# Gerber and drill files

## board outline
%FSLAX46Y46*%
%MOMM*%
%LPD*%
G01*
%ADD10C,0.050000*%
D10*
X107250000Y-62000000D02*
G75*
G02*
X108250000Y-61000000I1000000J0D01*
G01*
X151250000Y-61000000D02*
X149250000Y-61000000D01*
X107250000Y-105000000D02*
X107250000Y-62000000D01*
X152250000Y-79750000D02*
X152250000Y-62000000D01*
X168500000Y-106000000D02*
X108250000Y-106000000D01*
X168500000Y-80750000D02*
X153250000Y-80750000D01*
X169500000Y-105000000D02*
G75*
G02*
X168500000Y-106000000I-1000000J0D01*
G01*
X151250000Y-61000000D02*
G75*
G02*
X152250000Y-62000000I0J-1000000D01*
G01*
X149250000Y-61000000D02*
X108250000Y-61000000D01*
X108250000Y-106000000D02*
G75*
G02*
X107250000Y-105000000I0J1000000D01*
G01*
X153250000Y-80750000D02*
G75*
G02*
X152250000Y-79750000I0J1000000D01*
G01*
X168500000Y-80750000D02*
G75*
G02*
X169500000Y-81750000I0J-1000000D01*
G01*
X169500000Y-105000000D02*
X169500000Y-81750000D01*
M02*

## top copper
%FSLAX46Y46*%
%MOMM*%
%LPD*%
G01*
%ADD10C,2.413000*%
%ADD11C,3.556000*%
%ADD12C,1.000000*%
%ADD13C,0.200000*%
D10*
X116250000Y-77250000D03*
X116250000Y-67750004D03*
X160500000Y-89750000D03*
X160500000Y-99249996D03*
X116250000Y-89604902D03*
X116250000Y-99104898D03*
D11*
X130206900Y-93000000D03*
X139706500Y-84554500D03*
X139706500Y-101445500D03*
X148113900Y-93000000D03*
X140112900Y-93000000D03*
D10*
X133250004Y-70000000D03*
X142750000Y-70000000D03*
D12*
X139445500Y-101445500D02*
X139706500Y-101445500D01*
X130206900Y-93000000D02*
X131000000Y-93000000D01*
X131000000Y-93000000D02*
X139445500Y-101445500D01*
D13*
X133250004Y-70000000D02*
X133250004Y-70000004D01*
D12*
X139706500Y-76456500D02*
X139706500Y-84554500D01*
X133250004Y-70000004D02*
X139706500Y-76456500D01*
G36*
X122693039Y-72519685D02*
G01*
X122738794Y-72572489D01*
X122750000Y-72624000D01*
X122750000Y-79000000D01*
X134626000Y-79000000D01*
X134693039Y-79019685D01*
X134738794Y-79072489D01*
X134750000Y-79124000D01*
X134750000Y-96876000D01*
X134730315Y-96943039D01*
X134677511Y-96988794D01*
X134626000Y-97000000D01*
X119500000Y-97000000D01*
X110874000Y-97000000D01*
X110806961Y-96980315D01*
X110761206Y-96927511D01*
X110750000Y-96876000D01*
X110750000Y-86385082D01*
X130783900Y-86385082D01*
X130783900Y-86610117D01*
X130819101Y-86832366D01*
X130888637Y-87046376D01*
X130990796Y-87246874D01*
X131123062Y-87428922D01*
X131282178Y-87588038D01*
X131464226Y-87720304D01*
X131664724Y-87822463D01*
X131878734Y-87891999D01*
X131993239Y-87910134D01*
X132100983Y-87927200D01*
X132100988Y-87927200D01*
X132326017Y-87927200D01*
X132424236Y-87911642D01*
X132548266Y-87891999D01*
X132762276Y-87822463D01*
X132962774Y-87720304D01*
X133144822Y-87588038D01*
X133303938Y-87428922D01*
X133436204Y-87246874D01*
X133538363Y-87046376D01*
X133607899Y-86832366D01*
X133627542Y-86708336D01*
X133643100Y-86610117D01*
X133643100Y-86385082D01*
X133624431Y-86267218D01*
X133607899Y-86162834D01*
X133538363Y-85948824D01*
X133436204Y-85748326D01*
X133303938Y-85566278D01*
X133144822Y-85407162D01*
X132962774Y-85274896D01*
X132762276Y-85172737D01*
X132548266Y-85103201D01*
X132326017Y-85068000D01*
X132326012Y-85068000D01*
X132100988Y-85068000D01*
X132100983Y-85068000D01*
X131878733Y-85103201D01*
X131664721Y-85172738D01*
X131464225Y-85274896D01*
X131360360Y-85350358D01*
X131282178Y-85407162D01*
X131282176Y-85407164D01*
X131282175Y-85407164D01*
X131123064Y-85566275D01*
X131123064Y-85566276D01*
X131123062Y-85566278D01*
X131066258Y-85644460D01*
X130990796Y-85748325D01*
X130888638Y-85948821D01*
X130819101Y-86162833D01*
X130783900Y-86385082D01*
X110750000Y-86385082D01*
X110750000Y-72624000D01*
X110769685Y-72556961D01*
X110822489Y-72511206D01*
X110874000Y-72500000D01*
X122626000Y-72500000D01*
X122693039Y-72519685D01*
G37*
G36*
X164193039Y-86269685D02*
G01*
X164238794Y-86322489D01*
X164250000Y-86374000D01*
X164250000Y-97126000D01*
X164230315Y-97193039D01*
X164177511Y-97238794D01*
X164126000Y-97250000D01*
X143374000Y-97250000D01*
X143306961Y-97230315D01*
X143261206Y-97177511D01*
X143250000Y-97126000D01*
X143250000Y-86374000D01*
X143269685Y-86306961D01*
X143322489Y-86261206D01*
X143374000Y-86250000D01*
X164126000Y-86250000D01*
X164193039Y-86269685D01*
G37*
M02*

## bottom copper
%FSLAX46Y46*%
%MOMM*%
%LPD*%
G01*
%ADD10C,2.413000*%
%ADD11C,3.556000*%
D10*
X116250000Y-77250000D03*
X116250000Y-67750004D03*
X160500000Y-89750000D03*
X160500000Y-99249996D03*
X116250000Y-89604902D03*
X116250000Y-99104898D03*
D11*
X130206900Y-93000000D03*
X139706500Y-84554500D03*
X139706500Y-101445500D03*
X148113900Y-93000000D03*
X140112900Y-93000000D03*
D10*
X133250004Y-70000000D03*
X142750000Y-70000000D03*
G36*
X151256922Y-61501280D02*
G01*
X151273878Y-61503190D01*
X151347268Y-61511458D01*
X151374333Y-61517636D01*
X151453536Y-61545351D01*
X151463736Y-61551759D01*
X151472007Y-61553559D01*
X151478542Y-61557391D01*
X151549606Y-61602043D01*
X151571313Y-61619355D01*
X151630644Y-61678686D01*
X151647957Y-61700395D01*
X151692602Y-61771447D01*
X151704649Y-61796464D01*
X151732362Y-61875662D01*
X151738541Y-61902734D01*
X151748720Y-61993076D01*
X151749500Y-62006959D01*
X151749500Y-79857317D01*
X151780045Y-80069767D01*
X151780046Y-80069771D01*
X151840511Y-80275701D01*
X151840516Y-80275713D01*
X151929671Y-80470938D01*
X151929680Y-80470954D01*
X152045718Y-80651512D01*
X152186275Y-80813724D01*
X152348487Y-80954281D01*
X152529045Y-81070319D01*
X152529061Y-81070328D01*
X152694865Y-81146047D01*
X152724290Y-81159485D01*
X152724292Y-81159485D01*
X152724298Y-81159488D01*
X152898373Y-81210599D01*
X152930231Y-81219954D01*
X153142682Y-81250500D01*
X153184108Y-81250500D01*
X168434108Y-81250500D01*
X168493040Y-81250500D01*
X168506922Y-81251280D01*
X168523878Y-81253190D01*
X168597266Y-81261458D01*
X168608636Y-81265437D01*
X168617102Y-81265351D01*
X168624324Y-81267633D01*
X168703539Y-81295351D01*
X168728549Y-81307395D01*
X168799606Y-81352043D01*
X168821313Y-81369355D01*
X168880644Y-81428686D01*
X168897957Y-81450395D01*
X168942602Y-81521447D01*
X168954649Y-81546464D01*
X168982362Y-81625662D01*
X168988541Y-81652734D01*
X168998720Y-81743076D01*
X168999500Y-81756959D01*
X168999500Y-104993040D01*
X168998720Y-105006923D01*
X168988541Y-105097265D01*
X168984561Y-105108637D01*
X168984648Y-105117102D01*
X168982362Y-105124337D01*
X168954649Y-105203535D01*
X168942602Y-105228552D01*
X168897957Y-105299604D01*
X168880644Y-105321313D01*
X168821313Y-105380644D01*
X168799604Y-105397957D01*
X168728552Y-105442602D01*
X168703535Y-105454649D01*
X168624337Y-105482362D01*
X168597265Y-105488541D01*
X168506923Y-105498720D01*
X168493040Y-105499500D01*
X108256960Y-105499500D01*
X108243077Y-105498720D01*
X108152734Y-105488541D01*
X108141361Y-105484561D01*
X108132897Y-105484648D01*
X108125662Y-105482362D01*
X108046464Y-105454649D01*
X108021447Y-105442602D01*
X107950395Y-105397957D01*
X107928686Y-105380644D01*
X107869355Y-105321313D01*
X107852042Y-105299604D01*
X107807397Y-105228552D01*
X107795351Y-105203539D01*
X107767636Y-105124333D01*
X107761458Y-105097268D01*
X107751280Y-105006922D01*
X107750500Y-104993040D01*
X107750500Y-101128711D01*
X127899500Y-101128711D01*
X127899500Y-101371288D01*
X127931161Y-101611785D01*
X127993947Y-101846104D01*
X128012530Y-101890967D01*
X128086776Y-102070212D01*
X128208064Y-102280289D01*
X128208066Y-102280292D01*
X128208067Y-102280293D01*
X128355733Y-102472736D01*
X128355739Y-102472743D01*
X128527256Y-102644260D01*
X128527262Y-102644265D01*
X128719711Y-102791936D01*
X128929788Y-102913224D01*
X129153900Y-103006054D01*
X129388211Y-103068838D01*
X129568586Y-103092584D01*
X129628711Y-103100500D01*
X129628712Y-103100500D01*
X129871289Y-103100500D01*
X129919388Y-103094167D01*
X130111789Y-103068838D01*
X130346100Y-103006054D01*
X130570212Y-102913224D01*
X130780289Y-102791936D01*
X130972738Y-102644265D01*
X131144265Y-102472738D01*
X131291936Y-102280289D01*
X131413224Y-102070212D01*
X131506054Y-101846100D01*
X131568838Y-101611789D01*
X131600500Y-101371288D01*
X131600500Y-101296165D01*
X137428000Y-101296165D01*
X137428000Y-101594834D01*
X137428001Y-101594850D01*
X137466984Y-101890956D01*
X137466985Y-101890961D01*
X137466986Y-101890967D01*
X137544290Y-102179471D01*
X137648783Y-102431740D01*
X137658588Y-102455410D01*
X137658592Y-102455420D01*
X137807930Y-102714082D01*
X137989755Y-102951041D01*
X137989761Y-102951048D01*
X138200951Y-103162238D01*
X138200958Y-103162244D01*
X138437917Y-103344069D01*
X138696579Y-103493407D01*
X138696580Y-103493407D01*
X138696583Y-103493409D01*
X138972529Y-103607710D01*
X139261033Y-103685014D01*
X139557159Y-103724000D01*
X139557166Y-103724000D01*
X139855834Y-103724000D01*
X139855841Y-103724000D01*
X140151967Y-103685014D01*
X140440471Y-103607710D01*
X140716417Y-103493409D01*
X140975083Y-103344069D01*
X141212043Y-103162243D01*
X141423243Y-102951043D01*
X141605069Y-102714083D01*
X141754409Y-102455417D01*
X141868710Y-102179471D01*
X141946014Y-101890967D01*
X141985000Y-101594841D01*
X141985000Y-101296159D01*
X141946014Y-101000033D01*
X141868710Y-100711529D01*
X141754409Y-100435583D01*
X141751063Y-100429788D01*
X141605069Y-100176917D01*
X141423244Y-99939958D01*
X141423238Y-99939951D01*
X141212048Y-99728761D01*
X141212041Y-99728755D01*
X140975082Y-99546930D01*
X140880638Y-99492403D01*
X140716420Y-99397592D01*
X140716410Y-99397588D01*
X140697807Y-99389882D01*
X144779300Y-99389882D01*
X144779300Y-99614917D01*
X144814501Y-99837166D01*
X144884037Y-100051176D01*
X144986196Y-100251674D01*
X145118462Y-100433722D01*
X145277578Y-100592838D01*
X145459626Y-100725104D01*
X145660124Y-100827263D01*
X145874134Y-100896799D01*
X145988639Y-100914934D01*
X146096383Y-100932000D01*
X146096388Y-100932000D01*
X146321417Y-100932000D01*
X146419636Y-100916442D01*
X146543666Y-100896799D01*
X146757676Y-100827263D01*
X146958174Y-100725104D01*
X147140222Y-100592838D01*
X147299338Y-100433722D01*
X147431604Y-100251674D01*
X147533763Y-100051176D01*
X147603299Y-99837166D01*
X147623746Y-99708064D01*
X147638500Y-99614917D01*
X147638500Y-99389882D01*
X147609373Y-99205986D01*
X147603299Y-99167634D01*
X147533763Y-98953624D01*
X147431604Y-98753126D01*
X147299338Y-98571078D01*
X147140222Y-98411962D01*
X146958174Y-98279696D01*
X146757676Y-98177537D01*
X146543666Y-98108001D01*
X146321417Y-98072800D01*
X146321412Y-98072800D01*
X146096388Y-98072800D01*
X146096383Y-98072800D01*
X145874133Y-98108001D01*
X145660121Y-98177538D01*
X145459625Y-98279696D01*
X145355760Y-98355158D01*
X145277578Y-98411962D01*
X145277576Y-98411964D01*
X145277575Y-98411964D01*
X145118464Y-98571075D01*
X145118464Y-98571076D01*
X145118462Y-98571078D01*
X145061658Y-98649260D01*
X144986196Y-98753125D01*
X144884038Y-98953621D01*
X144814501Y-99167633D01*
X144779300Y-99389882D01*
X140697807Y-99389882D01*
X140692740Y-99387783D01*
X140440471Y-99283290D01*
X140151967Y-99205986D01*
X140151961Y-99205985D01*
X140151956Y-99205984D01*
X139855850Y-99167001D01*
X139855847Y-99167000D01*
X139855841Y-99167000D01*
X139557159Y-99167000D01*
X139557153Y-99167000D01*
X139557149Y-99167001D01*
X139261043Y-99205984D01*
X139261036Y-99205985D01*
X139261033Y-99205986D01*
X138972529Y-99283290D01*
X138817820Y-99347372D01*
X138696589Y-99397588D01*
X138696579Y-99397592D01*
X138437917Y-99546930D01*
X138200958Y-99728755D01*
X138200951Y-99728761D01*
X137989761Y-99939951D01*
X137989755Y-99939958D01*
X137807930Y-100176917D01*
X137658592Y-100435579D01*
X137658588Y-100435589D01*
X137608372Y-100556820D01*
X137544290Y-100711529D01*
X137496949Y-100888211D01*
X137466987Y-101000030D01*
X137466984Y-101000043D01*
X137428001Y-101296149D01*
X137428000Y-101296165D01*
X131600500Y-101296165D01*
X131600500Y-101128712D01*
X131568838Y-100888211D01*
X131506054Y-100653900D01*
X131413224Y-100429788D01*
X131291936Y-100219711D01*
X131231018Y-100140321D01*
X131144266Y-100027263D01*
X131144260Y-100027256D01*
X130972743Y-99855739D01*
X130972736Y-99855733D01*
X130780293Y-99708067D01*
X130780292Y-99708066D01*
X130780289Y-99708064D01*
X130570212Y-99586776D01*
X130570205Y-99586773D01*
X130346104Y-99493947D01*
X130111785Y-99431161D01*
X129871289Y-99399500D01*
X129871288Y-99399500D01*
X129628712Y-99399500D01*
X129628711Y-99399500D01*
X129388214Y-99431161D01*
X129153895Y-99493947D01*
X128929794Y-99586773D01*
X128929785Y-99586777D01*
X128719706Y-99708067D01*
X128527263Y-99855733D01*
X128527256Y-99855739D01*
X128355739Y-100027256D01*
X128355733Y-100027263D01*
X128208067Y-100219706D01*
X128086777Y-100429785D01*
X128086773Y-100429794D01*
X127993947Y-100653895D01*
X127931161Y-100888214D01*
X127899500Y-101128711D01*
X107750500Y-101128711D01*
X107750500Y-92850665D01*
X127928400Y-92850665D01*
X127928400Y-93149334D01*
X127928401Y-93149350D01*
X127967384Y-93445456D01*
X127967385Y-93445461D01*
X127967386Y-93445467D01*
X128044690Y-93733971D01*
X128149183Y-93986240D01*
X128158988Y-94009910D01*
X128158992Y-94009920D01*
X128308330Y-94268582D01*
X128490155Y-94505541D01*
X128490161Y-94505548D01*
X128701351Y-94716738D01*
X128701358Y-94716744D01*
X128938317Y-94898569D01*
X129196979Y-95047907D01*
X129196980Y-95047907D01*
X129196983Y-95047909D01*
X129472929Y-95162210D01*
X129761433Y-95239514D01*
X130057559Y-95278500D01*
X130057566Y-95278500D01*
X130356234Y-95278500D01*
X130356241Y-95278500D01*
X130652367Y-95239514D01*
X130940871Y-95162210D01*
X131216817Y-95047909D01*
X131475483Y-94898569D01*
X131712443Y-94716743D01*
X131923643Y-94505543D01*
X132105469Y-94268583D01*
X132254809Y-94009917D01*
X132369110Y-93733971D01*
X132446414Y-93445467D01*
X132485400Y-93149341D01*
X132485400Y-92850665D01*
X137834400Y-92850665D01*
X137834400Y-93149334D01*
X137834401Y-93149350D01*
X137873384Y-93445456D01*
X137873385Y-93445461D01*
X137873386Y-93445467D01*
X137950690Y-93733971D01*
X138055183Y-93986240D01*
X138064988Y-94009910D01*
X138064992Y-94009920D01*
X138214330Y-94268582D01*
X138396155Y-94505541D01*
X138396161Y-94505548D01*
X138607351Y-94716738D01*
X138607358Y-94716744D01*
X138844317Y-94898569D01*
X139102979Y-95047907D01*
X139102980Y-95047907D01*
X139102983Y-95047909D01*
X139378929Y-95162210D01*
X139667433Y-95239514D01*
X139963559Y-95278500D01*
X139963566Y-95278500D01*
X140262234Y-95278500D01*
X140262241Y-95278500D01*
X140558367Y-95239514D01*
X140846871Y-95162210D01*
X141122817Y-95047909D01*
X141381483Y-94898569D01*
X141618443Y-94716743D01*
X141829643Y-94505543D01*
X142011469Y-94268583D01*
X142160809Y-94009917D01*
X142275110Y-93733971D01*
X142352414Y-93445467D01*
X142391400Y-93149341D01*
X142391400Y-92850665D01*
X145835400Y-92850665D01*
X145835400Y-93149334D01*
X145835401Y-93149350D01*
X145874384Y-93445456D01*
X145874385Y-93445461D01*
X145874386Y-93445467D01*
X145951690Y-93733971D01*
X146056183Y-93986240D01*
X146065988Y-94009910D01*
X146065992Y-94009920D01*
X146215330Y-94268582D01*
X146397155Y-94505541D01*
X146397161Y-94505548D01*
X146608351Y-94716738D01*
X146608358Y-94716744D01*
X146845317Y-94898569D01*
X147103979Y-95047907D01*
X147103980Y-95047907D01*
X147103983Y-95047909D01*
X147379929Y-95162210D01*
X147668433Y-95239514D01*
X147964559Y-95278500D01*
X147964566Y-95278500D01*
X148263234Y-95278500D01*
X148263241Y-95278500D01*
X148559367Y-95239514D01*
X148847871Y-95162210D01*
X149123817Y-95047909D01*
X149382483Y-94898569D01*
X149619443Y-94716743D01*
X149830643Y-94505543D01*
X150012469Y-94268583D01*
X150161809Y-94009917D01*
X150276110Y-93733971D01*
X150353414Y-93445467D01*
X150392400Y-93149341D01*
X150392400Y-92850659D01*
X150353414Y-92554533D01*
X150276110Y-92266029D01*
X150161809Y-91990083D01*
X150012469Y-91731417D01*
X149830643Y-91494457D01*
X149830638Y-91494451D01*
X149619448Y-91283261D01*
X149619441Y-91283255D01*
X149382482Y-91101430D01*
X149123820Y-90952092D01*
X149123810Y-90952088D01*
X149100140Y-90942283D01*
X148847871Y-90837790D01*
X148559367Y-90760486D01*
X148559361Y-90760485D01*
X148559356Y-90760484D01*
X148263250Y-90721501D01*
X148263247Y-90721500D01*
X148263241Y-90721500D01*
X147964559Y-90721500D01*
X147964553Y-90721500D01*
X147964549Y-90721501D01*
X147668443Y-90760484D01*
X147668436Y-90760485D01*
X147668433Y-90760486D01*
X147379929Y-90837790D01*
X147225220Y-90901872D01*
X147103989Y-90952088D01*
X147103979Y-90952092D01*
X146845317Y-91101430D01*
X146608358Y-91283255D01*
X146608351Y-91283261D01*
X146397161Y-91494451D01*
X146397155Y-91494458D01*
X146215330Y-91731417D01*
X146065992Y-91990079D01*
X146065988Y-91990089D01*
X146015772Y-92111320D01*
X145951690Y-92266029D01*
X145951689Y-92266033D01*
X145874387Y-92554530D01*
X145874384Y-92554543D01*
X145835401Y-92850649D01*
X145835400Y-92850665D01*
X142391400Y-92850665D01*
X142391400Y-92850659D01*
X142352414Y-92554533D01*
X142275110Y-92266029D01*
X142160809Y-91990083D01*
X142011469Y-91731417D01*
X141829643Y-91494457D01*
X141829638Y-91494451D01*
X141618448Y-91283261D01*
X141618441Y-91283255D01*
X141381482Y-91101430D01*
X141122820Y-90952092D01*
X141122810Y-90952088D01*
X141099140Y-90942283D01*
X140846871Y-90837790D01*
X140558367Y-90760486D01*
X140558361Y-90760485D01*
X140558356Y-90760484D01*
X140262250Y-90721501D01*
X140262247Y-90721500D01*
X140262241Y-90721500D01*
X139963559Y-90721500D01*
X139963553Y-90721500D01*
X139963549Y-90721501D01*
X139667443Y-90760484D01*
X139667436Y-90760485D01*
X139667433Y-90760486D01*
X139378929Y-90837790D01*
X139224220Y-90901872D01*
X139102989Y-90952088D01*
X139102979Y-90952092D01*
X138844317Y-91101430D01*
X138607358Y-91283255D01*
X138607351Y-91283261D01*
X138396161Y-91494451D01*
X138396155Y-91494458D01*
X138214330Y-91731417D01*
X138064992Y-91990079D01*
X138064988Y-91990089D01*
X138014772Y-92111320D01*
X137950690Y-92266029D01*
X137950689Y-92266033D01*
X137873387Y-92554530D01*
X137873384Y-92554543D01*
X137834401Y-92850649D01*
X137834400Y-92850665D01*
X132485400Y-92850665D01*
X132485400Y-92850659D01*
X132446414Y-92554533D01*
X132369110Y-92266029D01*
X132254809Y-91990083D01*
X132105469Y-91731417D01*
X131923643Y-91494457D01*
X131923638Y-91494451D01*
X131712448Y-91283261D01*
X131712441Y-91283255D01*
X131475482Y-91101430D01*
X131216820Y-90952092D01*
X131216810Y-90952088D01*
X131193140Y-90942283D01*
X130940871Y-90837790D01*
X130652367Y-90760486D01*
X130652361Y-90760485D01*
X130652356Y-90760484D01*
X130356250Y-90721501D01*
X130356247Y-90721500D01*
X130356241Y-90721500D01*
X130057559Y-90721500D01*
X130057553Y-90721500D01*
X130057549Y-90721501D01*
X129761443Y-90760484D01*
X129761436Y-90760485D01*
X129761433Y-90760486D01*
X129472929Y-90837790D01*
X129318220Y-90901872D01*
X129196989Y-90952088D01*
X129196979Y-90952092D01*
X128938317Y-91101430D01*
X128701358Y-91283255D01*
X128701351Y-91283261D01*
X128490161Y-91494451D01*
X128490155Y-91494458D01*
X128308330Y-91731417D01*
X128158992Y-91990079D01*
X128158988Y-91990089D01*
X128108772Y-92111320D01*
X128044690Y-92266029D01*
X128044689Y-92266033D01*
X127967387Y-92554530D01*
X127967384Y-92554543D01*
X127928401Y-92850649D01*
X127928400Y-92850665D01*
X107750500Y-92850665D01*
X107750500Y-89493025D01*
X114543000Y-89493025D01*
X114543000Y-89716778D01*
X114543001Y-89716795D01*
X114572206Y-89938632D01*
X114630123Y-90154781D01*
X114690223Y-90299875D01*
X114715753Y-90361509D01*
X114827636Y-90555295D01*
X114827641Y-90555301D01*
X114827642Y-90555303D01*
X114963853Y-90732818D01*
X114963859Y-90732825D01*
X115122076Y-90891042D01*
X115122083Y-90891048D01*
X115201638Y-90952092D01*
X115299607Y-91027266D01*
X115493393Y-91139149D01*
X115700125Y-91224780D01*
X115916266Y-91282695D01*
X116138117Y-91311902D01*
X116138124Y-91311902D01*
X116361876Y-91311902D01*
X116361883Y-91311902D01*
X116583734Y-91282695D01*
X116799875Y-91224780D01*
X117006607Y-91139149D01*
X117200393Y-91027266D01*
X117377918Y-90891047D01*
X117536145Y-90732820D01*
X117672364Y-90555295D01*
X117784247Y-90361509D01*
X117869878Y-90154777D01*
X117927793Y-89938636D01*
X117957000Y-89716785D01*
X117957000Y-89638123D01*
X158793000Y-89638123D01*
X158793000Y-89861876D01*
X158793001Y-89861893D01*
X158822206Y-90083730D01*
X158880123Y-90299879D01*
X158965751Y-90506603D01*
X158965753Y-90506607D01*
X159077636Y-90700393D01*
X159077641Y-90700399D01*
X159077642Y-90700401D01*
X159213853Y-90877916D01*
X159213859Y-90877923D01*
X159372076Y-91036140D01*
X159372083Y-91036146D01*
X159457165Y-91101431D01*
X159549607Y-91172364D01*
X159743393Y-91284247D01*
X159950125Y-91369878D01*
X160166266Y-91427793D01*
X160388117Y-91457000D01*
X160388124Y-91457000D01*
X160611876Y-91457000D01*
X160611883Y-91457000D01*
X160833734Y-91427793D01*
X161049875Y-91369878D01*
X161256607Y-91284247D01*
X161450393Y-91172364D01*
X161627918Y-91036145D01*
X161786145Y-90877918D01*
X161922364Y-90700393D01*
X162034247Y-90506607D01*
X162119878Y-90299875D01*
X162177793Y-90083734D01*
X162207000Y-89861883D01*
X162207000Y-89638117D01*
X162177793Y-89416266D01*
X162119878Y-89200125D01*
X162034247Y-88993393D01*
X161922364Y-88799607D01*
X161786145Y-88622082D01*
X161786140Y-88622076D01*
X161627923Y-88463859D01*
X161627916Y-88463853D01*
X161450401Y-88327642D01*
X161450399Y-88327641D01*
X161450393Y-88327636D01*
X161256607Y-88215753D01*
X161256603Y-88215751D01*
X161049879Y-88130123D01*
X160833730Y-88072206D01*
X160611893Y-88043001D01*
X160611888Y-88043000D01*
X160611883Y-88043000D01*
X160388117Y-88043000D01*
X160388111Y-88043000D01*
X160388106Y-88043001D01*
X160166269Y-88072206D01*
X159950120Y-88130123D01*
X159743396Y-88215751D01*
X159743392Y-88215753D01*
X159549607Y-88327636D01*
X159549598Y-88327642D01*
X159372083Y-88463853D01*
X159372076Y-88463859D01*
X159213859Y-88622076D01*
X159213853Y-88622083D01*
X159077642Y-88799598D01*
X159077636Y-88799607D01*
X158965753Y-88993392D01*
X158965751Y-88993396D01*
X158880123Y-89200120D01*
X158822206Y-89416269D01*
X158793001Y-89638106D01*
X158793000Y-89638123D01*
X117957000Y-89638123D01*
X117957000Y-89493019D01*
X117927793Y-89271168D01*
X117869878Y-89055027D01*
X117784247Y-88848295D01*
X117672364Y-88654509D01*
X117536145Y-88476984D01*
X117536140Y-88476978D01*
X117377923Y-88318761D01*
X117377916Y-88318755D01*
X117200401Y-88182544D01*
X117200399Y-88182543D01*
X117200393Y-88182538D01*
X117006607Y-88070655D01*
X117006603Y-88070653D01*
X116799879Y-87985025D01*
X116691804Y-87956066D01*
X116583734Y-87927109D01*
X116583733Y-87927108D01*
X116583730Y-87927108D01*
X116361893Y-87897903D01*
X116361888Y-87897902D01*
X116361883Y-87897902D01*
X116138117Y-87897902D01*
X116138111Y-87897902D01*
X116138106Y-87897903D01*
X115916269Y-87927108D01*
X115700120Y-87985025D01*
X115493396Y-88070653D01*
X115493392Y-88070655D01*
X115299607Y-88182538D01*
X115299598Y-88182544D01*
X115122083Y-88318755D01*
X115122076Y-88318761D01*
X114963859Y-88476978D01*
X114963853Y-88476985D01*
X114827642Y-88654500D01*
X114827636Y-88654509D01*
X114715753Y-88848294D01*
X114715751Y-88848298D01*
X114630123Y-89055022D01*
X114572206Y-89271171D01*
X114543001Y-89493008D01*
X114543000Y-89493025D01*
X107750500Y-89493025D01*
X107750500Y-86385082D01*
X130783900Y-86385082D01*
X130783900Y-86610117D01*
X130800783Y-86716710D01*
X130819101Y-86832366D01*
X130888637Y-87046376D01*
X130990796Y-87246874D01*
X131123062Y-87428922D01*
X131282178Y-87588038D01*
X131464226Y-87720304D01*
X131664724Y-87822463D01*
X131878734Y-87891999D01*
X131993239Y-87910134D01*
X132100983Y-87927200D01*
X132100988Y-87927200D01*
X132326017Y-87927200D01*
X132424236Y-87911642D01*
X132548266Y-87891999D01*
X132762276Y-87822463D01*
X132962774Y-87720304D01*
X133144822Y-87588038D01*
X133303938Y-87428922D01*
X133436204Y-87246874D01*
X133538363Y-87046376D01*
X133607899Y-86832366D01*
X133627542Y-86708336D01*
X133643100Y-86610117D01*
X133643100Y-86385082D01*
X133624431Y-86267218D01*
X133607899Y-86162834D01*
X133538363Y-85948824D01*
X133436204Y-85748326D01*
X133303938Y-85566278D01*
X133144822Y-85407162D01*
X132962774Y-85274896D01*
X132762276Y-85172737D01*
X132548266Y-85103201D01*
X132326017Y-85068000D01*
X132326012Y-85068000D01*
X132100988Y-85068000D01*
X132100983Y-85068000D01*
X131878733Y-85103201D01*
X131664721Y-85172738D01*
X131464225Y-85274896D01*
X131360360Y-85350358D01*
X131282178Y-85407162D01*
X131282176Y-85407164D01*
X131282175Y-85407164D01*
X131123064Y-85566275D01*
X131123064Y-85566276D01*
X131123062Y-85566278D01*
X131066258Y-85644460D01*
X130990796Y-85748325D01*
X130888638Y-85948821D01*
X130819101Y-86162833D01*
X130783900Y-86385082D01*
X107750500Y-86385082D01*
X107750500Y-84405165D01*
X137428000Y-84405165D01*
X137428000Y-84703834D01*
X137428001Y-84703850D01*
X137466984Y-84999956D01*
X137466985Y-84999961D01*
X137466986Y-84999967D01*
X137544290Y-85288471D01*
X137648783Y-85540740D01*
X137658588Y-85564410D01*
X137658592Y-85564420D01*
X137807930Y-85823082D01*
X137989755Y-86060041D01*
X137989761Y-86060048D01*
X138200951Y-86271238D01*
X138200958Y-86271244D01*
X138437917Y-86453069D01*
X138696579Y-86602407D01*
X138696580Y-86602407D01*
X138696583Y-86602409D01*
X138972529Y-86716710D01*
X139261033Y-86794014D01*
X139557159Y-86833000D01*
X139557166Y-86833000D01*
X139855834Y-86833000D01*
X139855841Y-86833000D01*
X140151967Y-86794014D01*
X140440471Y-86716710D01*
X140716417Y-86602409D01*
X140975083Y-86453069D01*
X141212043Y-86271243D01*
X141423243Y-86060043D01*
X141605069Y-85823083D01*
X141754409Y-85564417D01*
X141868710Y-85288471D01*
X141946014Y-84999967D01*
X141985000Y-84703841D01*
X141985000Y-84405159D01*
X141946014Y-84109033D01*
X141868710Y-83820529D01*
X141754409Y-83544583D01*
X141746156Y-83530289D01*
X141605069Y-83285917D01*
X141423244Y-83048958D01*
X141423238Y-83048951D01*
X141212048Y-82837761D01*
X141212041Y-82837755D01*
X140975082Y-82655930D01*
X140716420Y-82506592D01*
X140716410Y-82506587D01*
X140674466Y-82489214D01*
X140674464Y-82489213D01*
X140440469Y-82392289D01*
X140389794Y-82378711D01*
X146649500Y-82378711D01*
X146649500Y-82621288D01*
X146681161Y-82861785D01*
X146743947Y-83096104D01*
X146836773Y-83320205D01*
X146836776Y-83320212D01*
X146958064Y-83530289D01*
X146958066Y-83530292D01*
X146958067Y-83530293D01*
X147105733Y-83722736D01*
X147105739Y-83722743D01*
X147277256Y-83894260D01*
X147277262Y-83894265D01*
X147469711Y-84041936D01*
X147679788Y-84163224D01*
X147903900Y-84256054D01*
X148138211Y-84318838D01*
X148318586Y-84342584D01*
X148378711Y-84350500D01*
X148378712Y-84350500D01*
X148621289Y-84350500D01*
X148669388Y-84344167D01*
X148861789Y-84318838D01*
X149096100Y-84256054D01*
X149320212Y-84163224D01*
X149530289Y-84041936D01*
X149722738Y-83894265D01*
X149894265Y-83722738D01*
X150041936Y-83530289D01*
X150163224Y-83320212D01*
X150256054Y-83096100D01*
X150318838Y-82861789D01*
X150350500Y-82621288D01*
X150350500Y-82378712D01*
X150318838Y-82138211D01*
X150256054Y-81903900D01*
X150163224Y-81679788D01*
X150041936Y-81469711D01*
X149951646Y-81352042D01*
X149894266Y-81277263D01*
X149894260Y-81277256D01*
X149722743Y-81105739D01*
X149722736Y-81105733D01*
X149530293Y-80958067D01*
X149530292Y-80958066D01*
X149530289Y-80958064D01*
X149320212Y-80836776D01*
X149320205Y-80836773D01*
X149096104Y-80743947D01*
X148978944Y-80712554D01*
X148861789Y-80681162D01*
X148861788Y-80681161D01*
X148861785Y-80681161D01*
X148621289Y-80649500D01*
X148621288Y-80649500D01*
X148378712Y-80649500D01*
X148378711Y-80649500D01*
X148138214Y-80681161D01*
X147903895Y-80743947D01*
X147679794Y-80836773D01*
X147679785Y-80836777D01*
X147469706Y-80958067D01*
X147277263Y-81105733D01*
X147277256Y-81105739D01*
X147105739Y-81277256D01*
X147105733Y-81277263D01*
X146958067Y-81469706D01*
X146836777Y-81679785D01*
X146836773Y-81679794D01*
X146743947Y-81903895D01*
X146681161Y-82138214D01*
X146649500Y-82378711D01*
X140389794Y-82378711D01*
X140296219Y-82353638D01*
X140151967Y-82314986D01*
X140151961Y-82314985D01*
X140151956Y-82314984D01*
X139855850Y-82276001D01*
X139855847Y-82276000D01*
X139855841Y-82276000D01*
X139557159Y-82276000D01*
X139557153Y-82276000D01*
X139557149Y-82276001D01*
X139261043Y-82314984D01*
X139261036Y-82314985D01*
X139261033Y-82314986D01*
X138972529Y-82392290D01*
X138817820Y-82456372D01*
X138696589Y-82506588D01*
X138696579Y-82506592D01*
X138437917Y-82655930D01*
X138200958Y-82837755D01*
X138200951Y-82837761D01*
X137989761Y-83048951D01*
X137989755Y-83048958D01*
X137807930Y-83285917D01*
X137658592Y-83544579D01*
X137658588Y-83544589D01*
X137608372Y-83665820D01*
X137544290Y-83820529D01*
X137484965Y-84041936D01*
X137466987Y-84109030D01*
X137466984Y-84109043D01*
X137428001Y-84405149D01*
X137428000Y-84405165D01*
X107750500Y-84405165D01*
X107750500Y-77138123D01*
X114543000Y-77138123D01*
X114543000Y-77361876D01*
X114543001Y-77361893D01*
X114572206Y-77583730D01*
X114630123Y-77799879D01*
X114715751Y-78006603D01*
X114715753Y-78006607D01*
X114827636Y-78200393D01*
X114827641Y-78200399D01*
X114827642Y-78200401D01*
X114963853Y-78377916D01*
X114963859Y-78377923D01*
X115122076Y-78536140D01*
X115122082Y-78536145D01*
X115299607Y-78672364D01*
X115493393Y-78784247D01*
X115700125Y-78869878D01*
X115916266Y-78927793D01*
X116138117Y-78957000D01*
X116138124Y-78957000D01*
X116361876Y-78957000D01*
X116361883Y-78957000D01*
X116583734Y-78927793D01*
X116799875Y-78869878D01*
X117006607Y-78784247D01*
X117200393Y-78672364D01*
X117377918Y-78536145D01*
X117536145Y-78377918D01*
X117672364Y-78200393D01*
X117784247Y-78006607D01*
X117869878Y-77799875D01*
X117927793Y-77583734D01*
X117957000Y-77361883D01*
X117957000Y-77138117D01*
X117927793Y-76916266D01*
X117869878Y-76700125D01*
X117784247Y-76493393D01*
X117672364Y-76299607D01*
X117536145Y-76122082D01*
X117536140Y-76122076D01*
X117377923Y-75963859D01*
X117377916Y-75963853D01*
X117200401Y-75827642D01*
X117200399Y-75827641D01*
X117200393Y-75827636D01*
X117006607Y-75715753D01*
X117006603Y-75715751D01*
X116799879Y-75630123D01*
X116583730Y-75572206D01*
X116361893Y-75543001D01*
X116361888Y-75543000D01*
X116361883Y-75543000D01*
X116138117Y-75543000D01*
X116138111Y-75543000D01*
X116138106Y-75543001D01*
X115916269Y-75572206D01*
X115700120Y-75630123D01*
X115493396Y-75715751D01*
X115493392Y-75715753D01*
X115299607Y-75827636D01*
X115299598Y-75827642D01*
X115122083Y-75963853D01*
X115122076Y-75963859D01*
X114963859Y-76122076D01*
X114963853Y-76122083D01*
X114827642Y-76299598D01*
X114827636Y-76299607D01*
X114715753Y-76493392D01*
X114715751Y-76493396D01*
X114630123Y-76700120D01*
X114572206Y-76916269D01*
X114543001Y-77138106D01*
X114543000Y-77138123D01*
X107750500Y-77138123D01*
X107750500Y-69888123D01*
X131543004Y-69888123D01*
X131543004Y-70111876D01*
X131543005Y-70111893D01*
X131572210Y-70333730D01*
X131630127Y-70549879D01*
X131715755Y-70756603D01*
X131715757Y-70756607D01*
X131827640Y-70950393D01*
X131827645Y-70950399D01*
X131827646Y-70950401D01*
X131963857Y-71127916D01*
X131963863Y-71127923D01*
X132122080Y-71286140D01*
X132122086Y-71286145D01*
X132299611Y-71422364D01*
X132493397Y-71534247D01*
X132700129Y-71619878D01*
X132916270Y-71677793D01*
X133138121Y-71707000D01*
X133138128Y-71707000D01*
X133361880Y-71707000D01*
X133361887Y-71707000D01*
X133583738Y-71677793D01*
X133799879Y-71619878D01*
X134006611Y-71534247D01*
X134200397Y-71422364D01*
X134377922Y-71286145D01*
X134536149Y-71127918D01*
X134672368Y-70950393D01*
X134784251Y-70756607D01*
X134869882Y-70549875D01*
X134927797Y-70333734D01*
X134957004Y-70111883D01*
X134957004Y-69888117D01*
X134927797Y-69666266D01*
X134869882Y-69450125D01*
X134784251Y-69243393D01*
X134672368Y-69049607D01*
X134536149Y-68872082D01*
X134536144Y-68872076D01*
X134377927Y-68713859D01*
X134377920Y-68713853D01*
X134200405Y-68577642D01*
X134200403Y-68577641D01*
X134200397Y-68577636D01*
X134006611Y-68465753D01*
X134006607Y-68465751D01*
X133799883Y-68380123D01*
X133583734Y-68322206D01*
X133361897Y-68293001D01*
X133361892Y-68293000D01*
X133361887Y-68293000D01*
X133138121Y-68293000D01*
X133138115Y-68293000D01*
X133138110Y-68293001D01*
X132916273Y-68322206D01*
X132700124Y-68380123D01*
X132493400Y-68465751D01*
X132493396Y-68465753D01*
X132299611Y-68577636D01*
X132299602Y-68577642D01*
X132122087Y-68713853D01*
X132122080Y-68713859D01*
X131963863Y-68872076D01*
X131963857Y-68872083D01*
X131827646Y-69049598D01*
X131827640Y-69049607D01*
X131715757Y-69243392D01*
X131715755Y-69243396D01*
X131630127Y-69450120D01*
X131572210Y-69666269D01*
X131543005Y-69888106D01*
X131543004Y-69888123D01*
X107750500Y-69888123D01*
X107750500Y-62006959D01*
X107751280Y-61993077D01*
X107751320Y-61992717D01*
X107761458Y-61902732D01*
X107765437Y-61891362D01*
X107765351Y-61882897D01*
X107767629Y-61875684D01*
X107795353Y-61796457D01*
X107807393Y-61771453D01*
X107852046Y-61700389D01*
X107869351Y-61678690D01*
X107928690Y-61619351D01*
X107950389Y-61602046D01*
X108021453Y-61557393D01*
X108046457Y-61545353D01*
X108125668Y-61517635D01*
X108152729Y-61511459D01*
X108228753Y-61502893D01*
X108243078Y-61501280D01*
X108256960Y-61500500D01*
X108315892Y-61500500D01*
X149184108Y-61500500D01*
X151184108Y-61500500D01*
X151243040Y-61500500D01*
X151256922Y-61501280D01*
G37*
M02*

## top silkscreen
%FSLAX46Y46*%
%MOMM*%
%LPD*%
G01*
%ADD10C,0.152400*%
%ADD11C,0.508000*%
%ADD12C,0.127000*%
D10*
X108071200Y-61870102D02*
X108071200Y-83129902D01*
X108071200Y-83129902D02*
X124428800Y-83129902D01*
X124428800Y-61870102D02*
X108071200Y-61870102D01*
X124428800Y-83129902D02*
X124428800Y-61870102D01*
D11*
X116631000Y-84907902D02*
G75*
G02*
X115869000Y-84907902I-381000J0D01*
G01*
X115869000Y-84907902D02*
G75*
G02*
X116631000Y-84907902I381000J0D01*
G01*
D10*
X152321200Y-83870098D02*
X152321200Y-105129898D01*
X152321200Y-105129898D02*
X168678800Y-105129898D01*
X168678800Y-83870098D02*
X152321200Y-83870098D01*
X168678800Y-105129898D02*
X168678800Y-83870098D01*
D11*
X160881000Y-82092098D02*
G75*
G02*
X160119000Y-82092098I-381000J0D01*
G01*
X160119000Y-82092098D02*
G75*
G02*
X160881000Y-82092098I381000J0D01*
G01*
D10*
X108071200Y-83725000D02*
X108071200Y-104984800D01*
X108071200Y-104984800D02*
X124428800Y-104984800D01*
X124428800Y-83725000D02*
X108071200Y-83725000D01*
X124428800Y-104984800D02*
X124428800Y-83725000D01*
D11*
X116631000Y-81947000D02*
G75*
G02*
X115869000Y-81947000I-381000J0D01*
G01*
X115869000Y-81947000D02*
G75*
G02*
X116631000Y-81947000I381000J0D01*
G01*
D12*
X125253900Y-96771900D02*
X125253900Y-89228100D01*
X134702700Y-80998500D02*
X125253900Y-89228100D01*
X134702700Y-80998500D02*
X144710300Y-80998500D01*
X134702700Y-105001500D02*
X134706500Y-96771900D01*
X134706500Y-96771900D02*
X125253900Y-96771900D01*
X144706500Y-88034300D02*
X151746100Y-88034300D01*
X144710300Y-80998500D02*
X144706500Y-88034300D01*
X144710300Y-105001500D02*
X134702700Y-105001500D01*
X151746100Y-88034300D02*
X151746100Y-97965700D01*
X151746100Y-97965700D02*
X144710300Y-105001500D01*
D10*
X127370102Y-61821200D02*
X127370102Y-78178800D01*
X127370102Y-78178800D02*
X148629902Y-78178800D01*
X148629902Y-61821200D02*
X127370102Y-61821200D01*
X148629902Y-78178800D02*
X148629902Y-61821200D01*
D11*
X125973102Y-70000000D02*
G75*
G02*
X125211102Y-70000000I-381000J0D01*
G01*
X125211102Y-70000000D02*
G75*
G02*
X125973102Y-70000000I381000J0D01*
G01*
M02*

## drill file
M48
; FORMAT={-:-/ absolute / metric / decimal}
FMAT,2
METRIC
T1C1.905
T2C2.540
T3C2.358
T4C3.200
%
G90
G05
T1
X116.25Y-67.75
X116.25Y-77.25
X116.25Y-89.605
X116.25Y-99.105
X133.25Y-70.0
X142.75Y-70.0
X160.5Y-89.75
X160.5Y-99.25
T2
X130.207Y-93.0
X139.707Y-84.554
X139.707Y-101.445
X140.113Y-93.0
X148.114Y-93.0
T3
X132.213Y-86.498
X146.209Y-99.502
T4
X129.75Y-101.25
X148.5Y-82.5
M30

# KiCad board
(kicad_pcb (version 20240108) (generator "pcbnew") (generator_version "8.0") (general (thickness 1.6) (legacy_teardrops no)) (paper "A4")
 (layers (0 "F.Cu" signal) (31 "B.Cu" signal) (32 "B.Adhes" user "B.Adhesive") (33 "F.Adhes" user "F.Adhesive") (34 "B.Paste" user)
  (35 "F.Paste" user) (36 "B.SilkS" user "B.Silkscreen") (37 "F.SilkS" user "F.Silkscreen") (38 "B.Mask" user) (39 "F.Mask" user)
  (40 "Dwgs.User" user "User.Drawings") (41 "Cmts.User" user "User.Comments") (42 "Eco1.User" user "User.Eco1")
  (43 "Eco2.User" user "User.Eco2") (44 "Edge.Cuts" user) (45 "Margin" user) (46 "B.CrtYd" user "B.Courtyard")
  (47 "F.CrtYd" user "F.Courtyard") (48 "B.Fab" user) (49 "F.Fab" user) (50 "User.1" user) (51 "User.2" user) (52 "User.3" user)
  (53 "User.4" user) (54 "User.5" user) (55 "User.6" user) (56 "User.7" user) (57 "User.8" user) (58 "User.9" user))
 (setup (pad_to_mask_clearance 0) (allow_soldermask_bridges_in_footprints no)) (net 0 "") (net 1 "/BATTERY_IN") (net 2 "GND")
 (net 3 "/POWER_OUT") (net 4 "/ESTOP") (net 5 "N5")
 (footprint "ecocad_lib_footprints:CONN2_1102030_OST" (layer "F.Cu") (at 116.25 77.25 90)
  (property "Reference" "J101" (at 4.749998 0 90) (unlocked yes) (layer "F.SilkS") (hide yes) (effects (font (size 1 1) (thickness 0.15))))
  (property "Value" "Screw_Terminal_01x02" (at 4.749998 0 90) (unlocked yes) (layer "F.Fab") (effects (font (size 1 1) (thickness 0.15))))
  (fp_line (start 15.379898 -8.1788) (end -5.879902 -8.1788) (stroke (width 0.1524) (type solid)) (layer "F.SilkS"))
  (fp_line (start -5.879902 -8.1788) (end -5.879902 8.1788) (stroke (width 0.1524) (type solid)) (layer "F.SilkS"))
  (fp_line (start 15.379898 8.1788) (end 15.379898 -8.1788) (stroke (width 0.1524) (type solid)) (layer "F.SilkS"))
  (fp_line (start -5.879902 8.1788) (end 15.379898 8.1788) (stroke (width 0.1524) (type solid)) (layer "F.SilkS"))
  (fp_circle (center -7.657902 0) (end -7.276902 0) (stroke (width 0.508) (type solid)) (fill none) (layer "F.SilkS"))
  (pad "1" thru_hole circle (at 0 0 90) (size 2.413 2.413) (drill 1.905) (layers "*.Cu" "*.Mask") (remove_unused_layers no)
   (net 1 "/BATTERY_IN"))
  (pad "2" thru_hole circle (at 9.499996 0 90) (size 2.413 2.413) (drill 1.905) (layers "*.Cu" "*.Mask") (remove_unused_layers no)
   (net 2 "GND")))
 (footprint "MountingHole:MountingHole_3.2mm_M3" (layer "F.Cu") (at 129.75 101.25)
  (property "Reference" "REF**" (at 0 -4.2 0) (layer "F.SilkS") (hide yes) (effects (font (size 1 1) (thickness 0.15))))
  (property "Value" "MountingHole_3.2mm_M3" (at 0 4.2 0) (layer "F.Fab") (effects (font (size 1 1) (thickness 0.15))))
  (pad "" np_thru_hole circle (at 0 0) (size 3.2 3.2) (drill 3.2) (layers "*.Cu" "*.Mask")))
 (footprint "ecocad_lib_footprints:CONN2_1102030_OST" (layer "F.Cu") (at 160.5 89.75 -90)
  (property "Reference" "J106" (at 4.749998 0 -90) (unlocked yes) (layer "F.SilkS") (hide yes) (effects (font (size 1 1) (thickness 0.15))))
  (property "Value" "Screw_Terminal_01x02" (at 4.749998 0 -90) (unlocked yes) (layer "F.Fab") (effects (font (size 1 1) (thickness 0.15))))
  (fp_line (start -5.879902 8.1788) (end 15.379898 8.1788) (stroke (width 0.1524) (type solid)) (layer "F.SilkS"))
  (fp_line (start 15.379898 8.1788) (end 15.379898 -8.1788) (stroke (width 0.1524) (type solid)) (layer "F.SilkS"))
  (fp_line (start -5.879902 -8.1788) (end -5.879902 8.1788) (stroke (width 0.1524) (type solid)) (layer "F.SilkS"))
  (fp_line (start 15.379898 -8.1788) (end -5.879902 -8.1788) (stroke (width 0.1524) (type solid)) (layer "F.SilkS"))
  (fp_circle (center -7.657902 0) (end -7.276902 0) (stroke (width 0.508) (type solid)) (fill none) (layer "F.SilkS"))
  (pad "1" thru_hole circle (at 0 0 270) (size 2.413 2.413) (drill 1.905) (layers "*.Cu" "*.Mask") (remove_unused_layers no)
   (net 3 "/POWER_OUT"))
  (pad "2" thru_hole circle (at 9.499996 0 270) (size 2.413 2.413) (drill 1.905) (layers "*.Cu" "*.Mask") (remove_unused_layers no)
   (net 2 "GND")))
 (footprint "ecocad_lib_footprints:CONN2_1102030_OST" (layer "F.Cu") (at 116.25 89.604902 -90)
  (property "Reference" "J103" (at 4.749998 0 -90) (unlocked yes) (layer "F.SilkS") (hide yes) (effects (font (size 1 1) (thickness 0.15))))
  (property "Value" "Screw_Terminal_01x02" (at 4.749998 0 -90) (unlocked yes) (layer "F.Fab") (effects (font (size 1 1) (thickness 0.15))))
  (fp_line (start -5.879902 8.1788) (end 15.379898 8.1788) (stroke (width 0.1524) (type solid)) (layer "F.SilkS"))
  (fp_line (start 15.379898 8.1788) (end 15.379898 -8.1788) (stroke (width 0.1524) (type solid)) (layer "F.SilkS"))
  (fp_line (start -5.879902 -8.1788) (end -5.879902 8.1788) (stroke (width 0.1524) (type solid)) (layer "F.SilkS"))
  (fp_line (start 15.379898 -8.1788) (end -5.879902 -8.1788) (stroke (width 0.1524) (type solid)) (layer "F.SilkS"))
  (fp_circle (center -7.657902 0) (end -7.276902 0) (stroke (width 0.508) (type solid)) (fill none) (layer "F.SilkS"))
  (pad "1" thru_hole circle (at 0 0 270) (size 2.413 2.413) (drill 1.905) (layers "*.Cu" "*.Mask") (remove_unused_layers no)
   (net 1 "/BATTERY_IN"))
  (pad "2" thru_hole circle (at 9.499996 0 270) (size 2.413 2.413) (drill 1.905) (layers "*.Cu" "*.Mask") (remove_unused_layers no)
   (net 2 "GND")))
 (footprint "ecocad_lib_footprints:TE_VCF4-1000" (layer "F.Cu") (at 139.7065 93 180)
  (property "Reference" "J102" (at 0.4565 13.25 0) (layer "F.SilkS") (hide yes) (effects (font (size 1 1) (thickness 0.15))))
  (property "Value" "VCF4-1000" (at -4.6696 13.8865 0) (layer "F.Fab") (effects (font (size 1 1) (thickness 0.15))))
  (fp_line (start 14.4526 -3.7719) (end 14.4526 3.7719) (stroke (width 0.127) (type solid)) (layer "F.SilkS"))
  (fp_line (start 5.0038 12.0015) (end 14.4526 3.7719) (stroke (width 0.127) (type solid)) (layer "F.SilkS"))
  (fp_line (start 5.0038 12.0015) (end -5.0038 12.0015) (stroke (width 0.127) (type solid)) (layer "F.SilkS"))
  (fp_line (start 5.0038 -12.0015) (end 5 -3.7719) (stroke (width 0.127) (type solid)) (layer "F.SilkS"))
  (fp_line (start 5 -3.7719) (end 14.4526 -3.7719) (stroke (width 0.127) (type solid)) (layer "F.SilkS"))
  (fp_line (start -5 4.9657) (end -12.0396 4.9657) (stroke (width 0.127) (type solid)) (layer "F.SilkS"))
  (fp_line (start -5.0038 12.0015) (end -5 4.9657) (stroke (width 0.127) (type solid)) (layer "F.SilkS"))
  (fp_line (start -5.0038 -12.0015) (end 5.0038 -12.0015) (stroke (width 0.127) (type solid)) (layer "F.SilkS"))
  (fp_line (start -12.0396 4.9657) (end -12.0396 -4.9657) (stroke (width 0.127) (type solid)) (layer "F.SilkS"))
  (fp_line (start -12.0396 -4.9657) (end -5.0038 -12.0015) (stroke (width 0.127) (type solid)) (layer "F.SilkS"))
  (pad "" np_thru_hole circle (at -6.5024 -6.5024 180) (size 2.3582 2.3582) (drill 2.3582) (layers "*.Cu" "*.Mask"))
  (pad "" np_thru_hole circle (at 7.493 6.5024 180) (size 2.3582 2.3582) (drill 2.3582) (layers "*.Cu" "*.Mask"))
  (pad "30" thru_hole circle (at 9.4996 0 180) (size 3.556 3.556) (drill 2.54) (layers "*.Cu" "*.Mask") (remove_unused_layers no)
   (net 1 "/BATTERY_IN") (solder_mask_margin 0.102))
  (pad "85" thru_hole circle (at 0 8.4455 180) (size 3.556 3.556) (drill 2.54) (layers "*.Cu" "*.Mask") (remove_unused_layers no)
   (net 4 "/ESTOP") (solder_mask_margin 0.102))
  (pad "86" thru_hole circle (at 0 -8.4455 180) (size 3.556 3.556) (drill 2.54) (layers "*.Cu" "*.Mask") (remove_unused_layers no)
   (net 1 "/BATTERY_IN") (solder_mask_margin 0.102))
  (pad "87" thru_hole circle (at -8.4074 0 180) (size 3.556 3.556) (drill 2.54) (layers "*.Cu" "*.Mask") (remove_unused_layers no)
   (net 3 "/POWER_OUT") (solder_mask_margin 0.102))
  (pad "87A" thru_hole circle (at -0.4064 0 180) (size 3.556 3.556) (drill 2.54) (layers "*.Cu" "*.Mask") (remove_unused_layers no)
   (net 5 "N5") (solder_mask_margin 0.102)))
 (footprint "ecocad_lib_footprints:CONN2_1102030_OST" (layer "F.Cu") (at 133.250004 70)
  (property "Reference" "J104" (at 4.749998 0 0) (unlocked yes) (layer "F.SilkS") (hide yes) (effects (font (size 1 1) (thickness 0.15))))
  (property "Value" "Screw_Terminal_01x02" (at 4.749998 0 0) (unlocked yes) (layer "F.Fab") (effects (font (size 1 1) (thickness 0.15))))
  (fp_line (start -5.879902 -8.1788) (end -5.879902 8.1788) (stroke (width 0.1524) (type solid)) (layer "F.SilkS"))
  (fp_line (start -5.879902 8.1788) (end 15.379898 8.1788) (stroke (width 0.1524) (type solid)) (layer "F.SilkS"))
  (fp_line (start 15.379898 -8.1788) (end -5.879902 -8.1788) (stroke (width 0.1524) (type solid)) (layer "F.SilkS"))
  (fp_line (start 15.379898 8.1788) (end 15.379898 -8.1788) (stroke (width 0.1524) (type solid)) (layer "F.SilkS"))
  (fp_circle (center -7.657902 0) (end -7.276902 0) (stroke (width 0.508) (type solid)) (fill none) (layer "F.SilkS"))
  (pad "1" thru_hole circle (at 0 0) (size 2.413 2.413) (drill 1.905) (layers "*.Cu" "*.Mask") (remove_unused_layers no) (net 4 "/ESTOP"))
  (pad "2" thru_hole circle (at 9.499996 0) (size 2.413 2.413) (drill 1.905) (layers "*.Cu" "*.Mask") (remove_unused_layers no)
   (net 2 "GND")))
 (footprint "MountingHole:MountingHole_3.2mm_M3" (layer "F.Cu") (at 148.5 82.5)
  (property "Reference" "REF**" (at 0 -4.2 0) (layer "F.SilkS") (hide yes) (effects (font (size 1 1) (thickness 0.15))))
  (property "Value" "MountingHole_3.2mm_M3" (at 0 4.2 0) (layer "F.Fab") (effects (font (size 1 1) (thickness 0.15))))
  (pad "" np_thru_hole circle (at 0 0) (size 3.2 3.2) (drill 3.2) (layers "*.Cu" "*.Mask")))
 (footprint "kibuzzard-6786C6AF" (layer "B.Cu") (at 116.25 94.5 -90)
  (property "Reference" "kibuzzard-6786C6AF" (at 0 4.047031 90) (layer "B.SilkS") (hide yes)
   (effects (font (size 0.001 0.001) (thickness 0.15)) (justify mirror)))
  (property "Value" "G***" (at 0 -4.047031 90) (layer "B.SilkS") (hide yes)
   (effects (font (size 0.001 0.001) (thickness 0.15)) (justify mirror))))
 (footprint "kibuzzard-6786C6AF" (layer "B.Cu") (at 160.5 94.75 -90)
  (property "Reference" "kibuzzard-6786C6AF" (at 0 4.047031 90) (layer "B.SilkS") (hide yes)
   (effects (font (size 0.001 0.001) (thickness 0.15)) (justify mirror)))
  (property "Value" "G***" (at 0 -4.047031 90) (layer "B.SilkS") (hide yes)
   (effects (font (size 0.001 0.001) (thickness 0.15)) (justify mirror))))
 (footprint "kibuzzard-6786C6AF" (layer "B.Cu") (at 116.25 72.25 90)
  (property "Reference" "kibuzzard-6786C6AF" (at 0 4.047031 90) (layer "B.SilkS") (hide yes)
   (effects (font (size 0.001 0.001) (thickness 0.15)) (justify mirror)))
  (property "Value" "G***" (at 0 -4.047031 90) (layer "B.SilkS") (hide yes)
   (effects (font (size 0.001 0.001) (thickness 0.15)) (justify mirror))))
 (gr_arc (start 107.25 62) (mid 107.542893 61.292893) (end 108.25 61) (stroke (width 0.05) (type default)) (layer "Edge.Cuts"))
 (gr_line (start 151.25 61) (end 149.25 61) (stroke (width 0.05) (type default)) (layer "Edge.Cuts"))
 (gr_line (start 107.25 105) (end 107.25 62) (stroke (width 0.05) (type default)) (layer "Edge.Cuts"))
 (gr_line (start 152.25 79.75) (end 152.25 62) (stroke (width 0.05) (type default)) (layer "Edge.Cuts"))
 (gr_line (start 168.5 106) (end 108.25 106) (stroke (width 0.05) (type default)) (layer "Edge.Cuts"))
 (gr_line (start 168.5 80.75) (end 153.25 80.75) (stroke (width 0.05) (type default)) (layer "Edge.Cuts"))
 (gr_arc (start 169.5 105) (mid 169.207107 105.707107) (end 168.5 106) (stroke (width 0.05) (type default)) (layer "Edge.Cuts"))
 (gr_arc (start 151.25 61) (mid 151.957107 61.292893) (end 152.25 62) (stroke (width 0.05) (type default)) (layer "Edge.Cuts"))
 (gr_line (start 149.25 61) (end 108.25 61) (stroke (width 0.05) (type default)) (layer "Edge.Cuts"))
 (gr_arc (start 108.25 106) (mid 107.542893 105.707107) (end 107.25 105) (stroke (width 0.05) (type default)) (layer "Edge.Cuts"))
 (gr_arc (start 153.25 80.75) (mid 152.542893 80.457107) (end 152.25 79.75) (stroke (width 0.05) (type default)) (layer "Edge.Cuts"))
 (gr_arc (start 168.5 80.75) (mid 169.207107 81.042893) (end 169.5 81.75) (stroke (width 0.05) (type default)) (layer "Edge.Cuts"))
 (gr_line (start 169.5 105) (end 169.5 81.75) (stroke (width 0.05) (type default)) (layer "Edge.Cuts"))
 (segment (start 139.4455 101.4455) (end 139.7065 101.4455) (width 1) (layer "F.Cu") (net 1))
 (segment (start 130.2069 93) (end 131 93) (width 1) (layer "F.Cu") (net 1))
 (segment (start 131 93) (end 139.4455 101.4455) (width 1) (layer "F.Cu") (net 1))
 (segment (start 133.250004 70) (end 133.250004 70.000004) (width 0.2) (layer "F.Cu") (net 4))
 (segment (start 139.7065 76.4565) (end 139.7065 84.5545) (width 1) (layer "F.Cu") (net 4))
 (segment (start 133.250004 70.000004) (end 139.7065 76.4565) (width 1) (layer "F.Cu") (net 4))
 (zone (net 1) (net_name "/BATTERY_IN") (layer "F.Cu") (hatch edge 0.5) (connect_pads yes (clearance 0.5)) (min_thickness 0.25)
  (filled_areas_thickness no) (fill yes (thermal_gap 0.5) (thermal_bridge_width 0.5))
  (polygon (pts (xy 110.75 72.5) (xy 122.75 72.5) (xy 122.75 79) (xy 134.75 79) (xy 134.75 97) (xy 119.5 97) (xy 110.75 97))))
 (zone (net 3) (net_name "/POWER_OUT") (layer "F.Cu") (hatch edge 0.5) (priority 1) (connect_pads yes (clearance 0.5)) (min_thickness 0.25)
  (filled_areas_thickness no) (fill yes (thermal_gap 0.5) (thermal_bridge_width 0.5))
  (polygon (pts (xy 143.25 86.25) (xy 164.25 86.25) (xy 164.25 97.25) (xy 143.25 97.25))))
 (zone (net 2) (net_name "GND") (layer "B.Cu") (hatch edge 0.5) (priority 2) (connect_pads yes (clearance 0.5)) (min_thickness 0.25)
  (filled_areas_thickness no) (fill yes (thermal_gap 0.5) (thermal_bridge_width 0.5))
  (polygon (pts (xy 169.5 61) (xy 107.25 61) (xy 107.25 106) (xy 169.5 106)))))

